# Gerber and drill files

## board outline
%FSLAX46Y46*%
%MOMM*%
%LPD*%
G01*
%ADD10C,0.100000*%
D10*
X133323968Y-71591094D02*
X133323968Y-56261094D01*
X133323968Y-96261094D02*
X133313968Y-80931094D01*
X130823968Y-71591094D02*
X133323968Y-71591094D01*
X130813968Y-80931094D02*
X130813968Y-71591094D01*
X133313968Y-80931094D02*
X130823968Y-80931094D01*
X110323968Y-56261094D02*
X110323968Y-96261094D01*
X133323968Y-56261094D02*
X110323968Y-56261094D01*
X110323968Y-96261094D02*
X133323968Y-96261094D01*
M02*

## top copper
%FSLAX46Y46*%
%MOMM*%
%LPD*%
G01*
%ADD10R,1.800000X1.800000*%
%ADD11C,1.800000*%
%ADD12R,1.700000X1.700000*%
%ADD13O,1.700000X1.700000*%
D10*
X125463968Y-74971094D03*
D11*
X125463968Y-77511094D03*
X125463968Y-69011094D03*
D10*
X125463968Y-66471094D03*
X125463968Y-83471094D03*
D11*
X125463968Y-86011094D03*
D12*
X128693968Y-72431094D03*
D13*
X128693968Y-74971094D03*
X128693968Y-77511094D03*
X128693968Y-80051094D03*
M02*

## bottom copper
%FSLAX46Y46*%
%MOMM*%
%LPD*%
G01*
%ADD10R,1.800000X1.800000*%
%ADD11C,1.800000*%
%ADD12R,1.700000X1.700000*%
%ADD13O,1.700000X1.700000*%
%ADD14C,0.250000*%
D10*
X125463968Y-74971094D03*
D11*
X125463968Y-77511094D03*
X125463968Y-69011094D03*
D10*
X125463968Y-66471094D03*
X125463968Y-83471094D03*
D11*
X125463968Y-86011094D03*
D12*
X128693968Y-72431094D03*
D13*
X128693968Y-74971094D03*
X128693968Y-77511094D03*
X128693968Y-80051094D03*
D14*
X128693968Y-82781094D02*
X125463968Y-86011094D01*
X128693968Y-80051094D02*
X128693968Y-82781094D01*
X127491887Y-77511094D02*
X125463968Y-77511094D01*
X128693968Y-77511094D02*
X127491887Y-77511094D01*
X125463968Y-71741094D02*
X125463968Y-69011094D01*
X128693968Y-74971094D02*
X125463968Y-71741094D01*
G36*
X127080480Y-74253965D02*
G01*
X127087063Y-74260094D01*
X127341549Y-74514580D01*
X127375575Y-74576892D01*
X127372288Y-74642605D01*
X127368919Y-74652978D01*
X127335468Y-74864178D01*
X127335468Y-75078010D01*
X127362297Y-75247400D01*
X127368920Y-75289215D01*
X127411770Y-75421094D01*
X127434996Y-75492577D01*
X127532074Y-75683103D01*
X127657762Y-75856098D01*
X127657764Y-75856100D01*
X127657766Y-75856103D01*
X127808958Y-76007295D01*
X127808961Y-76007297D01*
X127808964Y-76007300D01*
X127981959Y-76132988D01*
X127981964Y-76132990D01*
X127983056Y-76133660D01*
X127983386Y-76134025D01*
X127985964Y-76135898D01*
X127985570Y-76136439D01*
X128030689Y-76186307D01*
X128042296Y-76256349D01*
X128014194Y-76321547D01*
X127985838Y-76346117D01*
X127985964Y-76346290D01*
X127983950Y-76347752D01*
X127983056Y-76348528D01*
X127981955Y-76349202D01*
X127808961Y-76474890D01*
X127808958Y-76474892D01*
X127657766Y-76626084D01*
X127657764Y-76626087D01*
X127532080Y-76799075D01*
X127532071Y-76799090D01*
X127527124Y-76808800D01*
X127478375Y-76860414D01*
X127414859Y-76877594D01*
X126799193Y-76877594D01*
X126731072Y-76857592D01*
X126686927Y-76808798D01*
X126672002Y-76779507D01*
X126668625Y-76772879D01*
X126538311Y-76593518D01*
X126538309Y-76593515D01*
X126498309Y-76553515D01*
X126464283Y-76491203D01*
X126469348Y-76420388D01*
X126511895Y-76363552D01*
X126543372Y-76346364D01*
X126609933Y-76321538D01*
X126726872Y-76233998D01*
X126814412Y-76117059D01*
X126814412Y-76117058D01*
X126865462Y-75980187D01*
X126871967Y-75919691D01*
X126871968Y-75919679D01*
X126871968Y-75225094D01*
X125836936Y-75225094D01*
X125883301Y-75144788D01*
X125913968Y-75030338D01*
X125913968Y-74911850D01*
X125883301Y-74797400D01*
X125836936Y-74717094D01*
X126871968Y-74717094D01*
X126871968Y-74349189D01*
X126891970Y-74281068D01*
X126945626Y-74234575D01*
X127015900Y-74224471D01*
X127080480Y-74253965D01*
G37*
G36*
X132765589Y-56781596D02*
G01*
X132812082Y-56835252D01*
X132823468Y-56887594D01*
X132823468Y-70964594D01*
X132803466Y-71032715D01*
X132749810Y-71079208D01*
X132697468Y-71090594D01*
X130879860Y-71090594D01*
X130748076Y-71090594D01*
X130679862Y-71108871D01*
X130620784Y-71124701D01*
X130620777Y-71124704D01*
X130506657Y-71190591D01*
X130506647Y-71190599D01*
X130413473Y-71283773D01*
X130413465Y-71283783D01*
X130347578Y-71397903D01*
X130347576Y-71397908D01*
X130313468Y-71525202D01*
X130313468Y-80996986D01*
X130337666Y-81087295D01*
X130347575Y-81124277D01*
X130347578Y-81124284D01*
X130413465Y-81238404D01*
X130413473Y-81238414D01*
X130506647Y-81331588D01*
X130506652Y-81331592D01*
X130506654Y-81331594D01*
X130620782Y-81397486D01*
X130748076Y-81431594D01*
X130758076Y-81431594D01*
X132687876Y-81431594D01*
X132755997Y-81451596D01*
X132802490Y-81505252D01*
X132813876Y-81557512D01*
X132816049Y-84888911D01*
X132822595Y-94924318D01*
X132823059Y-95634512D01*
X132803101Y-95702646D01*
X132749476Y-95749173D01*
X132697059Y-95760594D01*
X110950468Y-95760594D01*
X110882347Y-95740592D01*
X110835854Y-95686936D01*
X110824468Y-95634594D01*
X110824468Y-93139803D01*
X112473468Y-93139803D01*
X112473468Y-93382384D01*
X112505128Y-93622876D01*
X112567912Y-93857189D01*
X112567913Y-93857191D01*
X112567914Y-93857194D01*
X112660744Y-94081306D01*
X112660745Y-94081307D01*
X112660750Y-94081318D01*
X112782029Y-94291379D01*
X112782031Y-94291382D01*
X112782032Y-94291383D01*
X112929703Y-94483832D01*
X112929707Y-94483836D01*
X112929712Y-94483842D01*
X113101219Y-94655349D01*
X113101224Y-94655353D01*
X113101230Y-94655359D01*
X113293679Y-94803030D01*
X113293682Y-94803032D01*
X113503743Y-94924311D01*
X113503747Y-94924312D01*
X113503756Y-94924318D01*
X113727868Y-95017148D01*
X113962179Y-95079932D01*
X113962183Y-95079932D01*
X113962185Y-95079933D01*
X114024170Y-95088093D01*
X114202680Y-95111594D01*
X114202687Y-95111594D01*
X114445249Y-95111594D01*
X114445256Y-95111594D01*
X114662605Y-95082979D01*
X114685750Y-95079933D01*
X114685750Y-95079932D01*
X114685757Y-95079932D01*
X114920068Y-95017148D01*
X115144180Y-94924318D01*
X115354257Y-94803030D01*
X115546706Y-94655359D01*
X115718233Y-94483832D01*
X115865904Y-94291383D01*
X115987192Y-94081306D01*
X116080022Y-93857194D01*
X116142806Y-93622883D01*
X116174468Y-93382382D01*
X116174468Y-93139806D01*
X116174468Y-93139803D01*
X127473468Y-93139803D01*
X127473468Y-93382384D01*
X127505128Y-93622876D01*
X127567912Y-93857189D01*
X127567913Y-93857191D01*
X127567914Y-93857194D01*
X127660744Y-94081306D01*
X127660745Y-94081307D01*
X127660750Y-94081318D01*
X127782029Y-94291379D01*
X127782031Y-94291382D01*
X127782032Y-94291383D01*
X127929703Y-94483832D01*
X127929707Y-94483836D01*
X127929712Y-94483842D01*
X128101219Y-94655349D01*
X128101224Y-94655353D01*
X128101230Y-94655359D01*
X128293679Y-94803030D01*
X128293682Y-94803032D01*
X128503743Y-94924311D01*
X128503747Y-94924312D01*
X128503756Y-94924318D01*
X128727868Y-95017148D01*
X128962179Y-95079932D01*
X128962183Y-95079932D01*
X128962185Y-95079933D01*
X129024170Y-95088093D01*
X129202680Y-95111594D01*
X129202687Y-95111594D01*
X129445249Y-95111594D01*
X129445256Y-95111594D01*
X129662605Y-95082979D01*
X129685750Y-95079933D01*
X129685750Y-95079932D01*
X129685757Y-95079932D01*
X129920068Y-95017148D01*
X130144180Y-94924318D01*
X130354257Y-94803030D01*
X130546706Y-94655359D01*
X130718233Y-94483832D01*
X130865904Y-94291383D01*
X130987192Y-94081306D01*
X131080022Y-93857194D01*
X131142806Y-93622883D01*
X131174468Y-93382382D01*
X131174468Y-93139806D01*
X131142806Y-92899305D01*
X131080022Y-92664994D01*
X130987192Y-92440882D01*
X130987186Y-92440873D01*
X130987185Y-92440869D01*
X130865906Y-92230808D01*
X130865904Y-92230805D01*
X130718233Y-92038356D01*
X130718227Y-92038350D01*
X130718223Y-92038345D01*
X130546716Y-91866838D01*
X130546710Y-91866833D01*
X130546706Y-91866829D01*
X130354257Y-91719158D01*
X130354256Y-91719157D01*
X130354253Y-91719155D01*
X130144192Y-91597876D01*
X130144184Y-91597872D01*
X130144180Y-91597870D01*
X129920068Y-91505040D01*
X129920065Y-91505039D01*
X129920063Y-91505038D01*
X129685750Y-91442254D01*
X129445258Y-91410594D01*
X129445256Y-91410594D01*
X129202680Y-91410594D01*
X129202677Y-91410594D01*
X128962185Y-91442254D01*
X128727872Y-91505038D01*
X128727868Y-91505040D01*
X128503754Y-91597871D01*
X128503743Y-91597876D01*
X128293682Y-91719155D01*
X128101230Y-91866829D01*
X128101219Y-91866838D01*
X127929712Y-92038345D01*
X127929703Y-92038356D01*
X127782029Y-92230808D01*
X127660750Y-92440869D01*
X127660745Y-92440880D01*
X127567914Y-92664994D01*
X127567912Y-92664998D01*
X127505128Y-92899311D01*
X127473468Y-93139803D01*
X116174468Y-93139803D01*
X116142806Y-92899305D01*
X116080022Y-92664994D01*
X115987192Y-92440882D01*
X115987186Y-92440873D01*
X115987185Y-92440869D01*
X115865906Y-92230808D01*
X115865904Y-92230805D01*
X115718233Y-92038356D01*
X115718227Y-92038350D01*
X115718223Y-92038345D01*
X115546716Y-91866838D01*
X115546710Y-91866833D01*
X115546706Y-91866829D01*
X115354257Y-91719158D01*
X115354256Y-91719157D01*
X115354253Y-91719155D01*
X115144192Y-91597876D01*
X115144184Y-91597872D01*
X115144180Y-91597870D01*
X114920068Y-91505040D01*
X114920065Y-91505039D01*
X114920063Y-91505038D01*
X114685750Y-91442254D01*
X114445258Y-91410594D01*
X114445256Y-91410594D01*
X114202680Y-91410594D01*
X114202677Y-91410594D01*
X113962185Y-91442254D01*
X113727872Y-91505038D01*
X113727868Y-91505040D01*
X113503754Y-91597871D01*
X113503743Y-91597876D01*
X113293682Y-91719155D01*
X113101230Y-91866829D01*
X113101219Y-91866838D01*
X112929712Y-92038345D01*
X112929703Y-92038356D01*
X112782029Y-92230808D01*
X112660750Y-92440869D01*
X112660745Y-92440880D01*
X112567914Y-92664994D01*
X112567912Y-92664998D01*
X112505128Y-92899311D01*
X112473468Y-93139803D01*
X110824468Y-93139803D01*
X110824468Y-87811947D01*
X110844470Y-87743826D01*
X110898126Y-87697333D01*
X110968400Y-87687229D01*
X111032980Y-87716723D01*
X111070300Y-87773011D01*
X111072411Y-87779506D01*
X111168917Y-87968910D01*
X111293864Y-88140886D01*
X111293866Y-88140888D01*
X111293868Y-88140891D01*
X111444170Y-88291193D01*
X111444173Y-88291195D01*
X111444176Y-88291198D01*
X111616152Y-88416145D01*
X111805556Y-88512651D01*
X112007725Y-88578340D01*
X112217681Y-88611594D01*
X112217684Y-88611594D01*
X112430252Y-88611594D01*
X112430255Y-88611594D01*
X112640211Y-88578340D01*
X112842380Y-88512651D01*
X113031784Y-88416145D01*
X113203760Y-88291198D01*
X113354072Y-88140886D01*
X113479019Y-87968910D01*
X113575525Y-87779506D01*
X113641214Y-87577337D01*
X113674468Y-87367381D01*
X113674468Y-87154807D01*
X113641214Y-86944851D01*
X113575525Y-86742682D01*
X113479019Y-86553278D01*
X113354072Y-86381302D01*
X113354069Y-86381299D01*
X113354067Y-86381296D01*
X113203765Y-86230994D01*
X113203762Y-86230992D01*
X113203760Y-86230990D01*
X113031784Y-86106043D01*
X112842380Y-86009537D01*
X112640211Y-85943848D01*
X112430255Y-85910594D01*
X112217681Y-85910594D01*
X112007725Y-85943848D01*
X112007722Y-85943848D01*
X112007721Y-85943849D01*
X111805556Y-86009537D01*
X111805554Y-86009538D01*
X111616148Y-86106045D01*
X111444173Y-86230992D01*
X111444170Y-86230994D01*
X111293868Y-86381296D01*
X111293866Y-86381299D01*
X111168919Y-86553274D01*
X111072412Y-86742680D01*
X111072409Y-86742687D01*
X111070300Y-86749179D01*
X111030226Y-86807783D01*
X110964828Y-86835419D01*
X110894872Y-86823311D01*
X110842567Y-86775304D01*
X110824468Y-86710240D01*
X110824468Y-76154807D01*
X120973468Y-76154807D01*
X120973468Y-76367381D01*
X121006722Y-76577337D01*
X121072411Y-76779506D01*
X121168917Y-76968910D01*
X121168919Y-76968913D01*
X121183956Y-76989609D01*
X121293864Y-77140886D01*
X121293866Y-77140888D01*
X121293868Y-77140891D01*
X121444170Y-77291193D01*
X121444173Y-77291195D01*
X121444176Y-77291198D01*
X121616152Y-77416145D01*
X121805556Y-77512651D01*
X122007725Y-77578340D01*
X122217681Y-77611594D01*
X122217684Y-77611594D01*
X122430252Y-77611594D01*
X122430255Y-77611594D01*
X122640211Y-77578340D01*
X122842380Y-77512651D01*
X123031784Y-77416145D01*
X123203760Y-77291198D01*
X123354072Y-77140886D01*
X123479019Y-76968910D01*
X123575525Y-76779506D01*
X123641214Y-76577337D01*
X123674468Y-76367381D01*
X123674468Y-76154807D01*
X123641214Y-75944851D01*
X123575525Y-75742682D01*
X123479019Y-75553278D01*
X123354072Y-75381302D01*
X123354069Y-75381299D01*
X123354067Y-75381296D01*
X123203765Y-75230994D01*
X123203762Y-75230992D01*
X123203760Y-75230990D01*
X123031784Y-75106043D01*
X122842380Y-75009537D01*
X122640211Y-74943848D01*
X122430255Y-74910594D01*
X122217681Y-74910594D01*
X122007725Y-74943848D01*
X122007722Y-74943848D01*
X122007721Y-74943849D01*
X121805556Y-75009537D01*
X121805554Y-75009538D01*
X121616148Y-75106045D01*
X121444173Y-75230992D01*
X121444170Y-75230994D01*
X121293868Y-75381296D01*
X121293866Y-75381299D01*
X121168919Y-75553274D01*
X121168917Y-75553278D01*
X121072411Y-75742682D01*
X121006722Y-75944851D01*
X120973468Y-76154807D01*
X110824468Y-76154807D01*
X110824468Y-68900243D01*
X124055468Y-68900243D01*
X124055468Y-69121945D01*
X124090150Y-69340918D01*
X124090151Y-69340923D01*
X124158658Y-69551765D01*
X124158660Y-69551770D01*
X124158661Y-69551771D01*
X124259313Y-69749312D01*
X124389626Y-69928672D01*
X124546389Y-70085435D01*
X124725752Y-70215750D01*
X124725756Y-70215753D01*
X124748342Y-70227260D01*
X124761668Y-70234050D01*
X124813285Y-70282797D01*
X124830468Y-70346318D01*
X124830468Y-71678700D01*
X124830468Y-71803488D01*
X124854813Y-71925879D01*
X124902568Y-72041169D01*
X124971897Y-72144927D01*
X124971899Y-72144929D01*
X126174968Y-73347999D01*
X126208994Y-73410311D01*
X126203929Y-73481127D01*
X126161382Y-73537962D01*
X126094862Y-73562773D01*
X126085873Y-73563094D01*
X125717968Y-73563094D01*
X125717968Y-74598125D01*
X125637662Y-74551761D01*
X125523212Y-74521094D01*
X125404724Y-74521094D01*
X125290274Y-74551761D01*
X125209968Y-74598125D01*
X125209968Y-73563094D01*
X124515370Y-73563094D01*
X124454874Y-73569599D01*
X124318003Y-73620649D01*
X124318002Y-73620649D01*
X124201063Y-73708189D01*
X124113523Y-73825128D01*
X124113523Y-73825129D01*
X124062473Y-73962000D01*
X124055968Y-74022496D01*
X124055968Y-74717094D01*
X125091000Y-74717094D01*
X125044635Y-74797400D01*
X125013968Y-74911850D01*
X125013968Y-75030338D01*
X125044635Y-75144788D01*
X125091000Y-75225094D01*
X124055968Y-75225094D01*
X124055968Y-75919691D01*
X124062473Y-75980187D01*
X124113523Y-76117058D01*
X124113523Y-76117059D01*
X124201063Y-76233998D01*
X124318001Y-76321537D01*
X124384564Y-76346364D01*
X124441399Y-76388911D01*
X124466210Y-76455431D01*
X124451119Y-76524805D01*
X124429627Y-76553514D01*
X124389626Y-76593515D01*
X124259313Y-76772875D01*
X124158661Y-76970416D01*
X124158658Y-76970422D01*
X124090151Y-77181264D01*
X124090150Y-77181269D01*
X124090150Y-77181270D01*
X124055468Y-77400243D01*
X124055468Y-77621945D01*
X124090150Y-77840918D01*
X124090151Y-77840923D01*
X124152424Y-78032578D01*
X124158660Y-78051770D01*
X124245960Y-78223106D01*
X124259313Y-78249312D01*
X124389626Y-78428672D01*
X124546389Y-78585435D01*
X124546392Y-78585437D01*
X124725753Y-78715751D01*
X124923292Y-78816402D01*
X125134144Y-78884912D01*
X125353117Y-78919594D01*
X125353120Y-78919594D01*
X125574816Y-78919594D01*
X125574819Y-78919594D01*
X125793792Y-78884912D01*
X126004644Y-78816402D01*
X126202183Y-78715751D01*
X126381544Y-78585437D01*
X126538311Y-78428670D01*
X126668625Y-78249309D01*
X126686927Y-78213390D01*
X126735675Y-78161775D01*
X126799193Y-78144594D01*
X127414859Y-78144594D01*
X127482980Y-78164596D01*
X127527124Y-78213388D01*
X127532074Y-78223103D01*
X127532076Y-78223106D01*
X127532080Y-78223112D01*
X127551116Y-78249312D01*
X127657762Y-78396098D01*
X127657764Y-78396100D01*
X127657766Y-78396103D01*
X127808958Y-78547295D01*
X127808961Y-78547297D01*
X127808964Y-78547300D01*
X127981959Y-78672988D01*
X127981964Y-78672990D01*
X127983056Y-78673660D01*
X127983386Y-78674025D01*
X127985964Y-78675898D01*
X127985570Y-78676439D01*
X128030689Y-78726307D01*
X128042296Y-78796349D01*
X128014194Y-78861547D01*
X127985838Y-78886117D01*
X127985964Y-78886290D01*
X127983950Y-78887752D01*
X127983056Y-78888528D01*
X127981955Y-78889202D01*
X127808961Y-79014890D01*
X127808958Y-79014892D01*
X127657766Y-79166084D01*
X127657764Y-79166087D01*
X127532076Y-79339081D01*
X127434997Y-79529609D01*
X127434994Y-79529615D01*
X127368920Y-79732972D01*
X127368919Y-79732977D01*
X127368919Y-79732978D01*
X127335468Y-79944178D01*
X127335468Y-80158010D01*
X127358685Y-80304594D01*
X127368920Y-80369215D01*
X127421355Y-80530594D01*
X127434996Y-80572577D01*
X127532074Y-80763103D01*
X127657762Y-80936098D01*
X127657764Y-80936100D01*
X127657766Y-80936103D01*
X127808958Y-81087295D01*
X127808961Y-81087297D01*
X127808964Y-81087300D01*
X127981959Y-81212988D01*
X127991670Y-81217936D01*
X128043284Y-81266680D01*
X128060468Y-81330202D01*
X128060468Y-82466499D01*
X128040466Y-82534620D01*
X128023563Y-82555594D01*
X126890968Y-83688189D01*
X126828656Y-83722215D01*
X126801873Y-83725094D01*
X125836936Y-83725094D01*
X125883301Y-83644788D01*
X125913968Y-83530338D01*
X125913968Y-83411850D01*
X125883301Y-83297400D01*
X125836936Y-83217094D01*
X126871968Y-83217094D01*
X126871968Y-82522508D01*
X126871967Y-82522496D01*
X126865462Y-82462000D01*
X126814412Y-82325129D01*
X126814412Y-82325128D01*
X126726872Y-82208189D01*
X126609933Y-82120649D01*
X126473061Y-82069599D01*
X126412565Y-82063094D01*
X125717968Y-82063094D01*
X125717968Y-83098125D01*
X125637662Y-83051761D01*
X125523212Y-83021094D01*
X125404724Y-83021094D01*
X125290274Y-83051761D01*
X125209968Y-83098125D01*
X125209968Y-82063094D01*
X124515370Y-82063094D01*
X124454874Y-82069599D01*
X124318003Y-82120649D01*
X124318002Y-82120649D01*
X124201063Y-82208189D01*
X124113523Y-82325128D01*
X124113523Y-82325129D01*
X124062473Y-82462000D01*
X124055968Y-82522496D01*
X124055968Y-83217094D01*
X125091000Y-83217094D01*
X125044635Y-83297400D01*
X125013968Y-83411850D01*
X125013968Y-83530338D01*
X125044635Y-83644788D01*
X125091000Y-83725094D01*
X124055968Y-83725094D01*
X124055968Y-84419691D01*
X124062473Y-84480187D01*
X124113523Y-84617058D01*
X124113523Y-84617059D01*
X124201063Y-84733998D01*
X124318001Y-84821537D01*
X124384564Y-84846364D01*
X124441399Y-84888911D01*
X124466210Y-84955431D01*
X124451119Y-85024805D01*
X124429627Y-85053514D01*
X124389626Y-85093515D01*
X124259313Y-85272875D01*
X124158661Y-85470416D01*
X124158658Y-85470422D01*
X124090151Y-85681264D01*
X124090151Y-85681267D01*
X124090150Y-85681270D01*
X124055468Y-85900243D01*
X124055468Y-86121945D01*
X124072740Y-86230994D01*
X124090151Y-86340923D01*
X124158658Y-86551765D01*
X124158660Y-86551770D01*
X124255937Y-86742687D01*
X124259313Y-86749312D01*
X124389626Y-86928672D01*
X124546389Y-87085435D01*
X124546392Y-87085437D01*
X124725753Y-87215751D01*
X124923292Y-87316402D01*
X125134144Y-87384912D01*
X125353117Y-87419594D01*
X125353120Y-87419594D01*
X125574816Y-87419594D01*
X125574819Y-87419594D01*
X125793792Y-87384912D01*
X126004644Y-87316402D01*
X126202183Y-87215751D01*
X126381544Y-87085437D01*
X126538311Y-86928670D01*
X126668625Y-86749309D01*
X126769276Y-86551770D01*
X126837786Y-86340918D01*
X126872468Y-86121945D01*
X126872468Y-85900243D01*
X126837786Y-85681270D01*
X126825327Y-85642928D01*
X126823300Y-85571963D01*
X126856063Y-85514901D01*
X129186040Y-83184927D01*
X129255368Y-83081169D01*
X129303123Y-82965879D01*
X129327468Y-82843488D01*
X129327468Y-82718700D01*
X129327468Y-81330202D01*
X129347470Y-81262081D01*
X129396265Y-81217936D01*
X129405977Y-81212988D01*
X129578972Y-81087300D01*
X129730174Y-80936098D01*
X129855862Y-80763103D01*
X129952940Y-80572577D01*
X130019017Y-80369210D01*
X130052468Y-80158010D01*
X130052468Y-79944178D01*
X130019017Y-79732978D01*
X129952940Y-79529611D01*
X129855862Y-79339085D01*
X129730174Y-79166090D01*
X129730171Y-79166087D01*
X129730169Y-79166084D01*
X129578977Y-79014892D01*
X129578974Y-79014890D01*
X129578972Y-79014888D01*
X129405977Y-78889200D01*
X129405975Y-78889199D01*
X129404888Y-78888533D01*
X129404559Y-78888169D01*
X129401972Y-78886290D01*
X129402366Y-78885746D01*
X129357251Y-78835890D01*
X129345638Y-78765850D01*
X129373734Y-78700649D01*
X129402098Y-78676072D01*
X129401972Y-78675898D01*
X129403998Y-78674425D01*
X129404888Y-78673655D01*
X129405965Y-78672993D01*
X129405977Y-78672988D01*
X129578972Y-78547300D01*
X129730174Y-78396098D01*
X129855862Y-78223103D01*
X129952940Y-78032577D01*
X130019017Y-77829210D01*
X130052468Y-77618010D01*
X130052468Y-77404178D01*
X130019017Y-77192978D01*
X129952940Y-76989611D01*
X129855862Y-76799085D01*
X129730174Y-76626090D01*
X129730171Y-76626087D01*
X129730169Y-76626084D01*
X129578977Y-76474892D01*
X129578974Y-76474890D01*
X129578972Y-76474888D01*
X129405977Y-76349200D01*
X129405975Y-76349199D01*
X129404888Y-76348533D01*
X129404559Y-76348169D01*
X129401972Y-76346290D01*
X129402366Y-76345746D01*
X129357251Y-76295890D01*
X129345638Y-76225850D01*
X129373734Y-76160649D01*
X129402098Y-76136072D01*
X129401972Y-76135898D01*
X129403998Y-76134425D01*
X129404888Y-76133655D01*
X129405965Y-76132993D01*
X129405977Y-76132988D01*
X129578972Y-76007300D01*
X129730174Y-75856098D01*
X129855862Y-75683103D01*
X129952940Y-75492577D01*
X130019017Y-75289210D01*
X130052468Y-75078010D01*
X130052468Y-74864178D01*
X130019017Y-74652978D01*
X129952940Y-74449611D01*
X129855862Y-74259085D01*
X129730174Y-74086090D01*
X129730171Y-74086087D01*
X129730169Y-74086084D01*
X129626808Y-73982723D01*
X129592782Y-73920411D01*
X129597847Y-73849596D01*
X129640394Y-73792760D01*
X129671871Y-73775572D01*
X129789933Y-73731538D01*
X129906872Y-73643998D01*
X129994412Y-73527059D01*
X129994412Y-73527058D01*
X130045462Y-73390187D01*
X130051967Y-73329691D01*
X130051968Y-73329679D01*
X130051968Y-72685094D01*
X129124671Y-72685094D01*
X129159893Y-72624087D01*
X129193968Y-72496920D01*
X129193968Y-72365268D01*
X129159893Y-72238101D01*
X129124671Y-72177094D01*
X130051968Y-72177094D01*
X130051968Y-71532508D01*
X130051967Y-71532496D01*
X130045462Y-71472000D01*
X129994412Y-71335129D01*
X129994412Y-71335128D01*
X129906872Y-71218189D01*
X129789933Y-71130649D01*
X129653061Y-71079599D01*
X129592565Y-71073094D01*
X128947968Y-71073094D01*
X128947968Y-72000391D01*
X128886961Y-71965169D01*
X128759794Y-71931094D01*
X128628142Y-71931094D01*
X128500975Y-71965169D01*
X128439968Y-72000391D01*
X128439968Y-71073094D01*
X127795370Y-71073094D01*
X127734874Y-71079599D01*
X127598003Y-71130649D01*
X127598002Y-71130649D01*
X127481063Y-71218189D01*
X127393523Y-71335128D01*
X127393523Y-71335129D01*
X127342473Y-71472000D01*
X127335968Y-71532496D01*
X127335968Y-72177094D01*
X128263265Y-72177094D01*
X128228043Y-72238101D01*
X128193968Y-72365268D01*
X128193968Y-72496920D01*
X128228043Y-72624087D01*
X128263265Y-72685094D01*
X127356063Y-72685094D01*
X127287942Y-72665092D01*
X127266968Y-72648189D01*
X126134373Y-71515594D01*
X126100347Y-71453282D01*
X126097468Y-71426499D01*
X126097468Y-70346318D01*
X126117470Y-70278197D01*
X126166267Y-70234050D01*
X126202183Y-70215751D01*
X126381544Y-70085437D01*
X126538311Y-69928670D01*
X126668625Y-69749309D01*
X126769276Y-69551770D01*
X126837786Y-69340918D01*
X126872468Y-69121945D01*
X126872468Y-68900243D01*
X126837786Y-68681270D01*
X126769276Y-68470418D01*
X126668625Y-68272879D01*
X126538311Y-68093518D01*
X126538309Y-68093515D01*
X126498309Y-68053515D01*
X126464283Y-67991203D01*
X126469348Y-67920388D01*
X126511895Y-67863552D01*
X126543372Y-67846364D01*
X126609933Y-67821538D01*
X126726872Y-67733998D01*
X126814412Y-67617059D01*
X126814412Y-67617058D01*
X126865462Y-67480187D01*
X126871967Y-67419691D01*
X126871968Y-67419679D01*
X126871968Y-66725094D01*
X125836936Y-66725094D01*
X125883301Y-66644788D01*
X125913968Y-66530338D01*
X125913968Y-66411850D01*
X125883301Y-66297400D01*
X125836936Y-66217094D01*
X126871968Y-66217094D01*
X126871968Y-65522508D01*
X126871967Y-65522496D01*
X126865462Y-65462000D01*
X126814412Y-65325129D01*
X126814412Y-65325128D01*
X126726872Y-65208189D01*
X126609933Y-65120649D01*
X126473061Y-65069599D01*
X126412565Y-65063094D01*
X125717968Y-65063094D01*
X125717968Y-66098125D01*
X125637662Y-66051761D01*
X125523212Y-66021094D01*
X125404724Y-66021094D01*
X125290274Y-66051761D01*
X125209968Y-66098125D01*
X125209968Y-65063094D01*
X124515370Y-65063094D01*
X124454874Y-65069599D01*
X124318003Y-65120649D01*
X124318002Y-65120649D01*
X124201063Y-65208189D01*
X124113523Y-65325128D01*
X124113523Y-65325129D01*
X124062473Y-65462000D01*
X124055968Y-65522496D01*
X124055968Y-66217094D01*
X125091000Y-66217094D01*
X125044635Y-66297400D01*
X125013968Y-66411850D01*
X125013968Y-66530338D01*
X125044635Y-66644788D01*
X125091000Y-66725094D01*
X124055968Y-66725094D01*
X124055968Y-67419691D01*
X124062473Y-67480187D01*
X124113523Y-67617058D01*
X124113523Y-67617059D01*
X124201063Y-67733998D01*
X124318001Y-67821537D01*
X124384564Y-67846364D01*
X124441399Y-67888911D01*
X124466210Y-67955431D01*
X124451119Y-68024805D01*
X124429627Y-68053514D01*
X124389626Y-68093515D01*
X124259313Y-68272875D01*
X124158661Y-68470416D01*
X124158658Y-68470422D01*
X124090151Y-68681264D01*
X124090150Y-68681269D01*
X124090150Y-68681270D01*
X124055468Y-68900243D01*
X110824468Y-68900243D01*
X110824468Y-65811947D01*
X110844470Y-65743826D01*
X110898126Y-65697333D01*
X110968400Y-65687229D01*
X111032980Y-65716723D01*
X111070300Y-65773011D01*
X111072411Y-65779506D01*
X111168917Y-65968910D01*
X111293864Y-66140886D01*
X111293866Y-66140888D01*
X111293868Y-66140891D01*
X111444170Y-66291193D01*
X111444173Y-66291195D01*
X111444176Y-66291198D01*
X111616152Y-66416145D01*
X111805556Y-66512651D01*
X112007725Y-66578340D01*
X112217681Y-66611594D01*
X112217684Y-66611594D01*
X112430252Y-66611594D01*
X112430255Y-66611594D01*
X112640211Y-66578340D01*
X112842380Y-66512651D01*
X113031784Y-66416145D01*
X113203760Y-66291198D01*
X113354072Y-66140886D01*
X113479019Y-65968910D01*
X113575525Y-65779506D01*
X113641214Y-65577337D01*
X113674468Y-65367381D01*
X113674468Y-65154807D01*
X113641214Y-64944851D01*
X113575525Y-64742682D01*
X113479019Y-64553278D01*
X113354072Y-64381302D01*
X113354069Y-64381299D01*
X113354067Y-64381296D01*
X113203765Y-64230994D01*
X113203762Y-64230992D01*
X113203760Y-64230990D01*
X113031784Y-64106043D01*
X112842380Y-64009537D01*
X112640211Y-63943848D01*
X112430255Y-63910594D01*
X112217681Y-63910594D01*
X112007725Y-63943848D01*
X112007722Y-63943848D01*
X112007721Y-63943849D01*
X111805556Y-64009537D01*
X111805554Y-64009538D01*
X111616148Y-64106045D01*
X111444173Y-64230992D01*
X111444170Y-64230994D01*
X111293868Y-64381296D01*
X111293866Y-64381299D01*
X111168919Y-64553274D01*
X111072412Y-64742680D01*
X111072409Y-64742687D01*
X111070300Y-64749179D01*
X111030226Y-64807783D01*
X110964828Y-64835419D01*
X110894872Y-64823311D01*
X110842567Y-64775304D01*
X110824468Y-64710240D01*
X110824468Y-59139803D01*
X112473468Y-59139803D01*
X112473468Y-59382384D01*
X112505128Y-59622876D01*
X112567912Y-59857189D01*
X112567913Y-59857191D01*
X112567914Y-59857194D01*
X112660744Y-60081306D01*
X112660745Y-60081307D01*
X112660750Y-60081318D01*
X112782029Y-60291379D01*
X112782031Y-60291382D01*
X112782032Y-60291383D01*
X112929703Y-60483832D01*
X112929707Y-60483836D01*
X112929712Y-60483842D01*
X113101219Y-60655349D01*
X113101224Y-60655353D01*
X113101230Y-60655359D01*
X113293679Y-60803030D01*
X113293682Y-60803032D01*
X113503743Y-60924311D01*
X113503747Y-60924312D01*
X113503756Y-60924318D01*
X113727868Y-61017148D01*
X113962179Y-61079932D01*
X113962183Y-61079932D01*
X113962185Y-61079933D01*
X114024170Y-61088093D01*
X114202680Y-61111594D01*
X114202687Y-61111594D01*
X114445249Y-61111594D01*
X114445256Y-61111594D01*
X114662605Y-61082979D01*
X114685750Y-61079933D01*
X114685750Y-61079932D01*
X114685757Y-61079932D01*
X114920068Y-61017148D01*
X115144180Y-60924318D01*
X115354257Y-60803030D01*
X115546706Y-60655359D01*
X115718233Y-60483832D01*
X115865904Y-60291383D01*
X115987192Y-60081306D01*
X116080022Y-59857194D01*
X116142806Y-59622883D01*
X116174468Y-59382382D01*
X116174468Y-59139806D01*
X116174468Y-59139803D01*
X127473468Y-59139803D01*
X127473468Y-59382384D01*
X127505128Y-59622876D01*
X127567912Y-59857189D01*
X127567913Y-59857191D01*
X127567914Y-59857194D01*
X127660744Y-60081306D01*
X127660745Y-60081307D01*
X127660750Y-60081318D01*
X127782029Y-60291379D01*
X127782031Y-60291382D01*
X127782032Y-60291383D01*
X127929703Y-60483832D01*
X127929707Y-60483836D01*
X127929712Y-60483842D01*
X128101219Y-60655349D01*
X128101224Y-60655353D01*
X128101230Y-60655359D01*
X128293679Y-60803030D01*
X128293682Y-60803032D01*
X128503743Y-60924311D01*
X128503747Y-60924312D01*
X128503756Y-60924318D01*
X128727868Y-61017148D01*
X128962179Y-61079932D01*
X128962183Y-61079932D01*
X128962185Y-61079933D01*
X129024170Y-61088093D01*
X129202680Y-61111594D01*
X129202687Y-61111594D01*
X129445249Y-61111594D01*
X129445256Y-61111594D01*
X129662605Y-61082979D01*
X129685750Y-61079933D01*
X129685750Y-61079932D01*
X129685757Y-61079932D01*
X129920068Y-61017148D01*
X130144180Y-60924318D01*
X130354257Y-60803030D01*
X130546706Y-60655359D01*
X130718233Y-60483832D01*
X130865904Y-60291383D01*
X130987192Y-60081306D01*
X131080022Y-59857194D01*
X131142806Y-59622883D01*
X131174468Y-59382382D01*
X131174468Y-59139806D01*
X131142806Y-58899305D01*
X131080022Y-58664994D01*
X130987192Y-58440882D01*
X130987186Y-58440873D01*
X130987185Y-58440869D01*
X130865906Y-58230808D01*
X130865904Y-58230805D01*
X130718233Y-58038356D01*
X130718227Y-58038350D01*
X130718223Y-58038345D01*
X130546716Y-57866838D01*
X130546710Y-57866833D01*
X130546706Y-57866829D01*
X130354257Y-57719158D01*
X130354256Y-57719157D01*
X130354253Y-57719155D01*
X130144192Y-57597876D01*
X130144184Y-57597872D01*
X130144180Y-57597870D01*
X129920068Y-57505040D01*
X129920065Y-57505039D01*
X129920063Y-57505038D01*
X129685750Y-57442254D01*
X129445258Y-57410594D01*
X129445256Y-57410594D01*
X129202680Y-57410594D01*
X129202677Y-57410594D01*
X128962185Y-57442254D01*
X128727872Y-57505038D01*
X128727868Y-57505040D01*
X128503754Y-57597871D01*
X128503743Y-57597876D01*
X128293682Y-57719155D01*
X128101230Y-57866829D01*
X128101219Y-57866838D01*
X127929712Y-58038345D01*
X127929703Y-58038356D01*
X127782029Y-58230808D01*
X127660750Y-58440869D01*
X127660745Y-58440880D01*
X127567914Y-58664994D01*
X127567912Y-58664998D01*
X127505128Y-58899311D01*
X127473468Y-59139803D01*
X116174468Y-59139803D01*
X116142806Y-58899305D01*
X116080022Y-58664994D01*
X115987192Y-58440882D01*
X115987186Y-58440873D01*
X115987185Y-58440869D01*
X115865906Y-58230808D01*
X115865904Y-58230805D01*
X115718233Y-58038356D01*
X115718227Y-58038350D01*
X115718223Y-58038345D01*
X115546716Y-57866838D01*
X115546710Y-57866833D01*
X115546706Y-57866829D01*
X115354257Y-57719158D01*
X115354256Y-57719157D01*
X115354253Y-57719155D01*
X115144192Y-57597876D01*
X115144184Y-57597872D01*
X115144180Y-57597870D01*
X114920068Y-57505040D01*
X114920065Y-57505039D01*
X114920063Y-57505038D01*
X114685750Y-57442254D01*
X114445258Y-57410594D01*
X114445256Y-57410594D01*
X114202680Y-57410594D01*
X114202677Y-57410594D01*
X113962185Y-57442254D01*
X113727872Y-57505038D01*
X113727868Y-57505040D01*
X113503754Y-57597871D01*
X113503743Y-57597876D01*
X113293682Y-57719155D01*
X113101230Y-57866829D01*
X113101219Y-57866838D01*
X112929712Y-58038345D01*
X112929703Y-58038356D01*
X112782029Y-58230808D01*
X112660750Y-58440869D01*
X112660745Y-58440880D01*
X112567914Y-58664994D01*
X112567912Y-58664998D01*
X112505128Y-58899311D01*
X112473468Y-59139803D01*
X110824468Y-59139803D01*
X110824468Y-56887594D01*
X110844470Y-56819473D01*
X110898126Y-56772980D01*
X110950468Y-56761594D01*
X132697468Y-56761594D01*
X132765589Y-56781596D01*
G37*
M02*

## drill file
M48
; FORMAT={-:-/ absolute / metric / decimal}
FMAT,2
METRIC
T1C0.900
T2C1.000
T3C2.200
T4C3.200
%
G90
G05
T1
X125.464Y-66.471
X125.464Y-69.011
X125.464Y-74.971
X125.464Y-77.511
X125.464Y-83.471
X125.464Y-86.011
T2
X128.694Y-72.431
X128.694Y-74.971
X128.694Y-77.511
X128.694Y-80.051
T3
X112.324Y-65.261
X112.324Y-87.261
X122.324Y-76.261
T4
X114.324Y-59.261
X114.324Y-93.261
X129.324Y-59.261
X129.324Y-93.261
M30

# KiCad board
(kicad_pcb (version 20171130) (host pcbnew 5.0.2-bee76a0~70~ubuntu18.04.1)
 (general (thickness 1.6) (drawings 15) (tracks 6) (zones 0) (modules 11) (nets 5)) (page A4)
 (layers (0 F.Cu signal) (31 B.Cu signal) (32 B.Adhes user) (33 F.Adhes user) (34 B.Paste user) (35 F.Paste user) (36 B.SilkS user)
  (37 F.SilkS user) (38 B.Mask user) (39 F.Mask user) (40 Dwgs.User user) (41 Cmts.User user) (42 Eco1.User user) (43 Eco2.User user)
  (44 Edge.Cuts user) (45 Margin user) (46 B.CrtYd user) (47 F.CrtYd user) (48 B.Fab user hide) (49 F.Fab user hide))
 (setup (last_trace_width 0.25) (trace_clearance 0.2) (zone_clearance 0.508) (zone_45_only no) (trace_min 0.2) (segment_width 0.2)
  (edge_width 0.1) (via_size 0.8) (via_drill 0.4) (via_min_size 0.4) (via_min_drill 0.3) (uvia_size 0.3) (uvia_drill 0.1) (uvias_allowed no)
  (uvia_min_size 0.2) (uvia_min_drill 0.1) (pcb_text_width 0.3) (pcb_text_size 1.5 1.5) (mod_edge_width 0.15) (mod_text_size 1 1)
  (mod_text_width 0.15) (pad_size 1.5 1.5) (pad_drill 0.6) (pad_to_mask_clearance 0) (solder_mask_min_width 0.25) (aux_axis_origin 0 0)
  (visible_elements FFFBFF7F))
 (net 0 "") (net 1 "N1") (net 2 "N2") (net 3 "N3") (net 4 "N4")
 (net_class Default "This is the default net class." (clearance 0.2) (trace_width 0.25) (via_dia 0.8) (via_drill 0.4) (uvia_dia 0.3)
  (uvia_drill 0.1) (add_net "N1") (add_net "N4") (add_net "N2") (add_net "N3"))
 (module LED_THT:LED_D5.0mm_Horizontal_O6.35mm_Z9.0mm (layer F.Cu) (at 125.463968 74.971094 270)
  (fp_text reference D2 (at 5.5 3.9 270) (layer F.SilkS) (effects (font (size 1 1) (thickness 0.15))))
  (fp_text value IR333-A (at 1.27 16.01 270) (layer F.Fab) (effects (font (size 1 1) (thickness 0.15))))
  (pad 1 thru_hole rect (at 0 0 270) (size 1.8 1.8) (drill 0.9) (layers *.Cu *.Mask) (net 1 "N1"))
  (pad 2 thru_hole circle (at 2.54 0 270) (size 1.8 1.8) (drill 0.9) (layers *.Cu *.Mask) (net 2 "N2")))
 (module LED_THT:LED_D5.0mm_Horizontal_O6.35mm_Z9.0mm (layer F.Cu) (at 125.463968 66.471094 270)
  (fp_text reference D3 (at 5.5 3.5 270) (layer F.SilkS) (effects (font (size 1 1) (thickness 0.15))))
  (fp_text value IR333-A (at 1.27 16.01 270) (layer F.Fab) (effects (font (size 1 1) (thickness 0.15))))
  (pad 2 thru_hole circle (at 2.54 0 270) (size 1.8 1.8) (drill 0.9) (layers *.Cu *.Mask) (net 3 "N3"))
  (pad 1 thru_hole rect (at 0 0 270) (size 1.8 1.8) (drill 0.9) (layers *.Cu *.Mask) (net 1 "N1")))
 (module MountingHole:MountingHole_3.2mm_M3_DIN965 (layer F.Cu) (at 129.323968 59.261094 180)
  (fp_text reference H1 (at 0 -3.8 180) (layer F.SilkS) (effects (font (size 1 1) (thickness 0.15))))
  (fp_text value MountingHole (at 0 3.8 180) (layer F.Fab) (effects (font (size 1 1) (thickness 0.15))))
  (pad 1 np_thru_hole circle (at 0 0 180) (size 3.2 3.2) (drill 3.2) (layers *.Cu *.Mask)))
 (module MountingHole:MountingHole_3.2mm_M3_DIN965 (layer F.Cu) (at 129.323968 93.261094 180)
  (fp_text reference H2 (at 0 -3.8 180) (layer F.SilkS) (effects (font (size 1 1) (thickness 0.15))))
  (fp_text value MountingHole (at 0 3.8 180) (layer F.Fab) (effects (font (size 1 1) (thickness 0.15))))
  (pad 1 np_thru_hole circle (at 0 0 180) (size 3.2 3.2) (drill 3.2) (layers *.Cu *.Mask)))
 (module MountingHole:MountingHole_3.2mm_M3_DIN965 (layer F.Cu) (at 114.323968 59.261094 180)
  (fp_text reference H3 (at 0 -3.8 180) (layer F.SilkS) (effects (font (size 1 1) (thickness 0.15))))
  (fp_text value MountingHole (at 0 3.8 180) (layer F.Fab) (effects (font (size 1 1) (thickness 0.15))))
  (pad 1 np_thru_hole circle (at 0 0 180) (size 3.2 3.2) (drill 3.2) (layers *.Cu *.Mask)))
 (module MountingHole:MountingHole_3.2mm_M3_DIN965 (layer F.Cu) (at 114.323968 93.261094 180)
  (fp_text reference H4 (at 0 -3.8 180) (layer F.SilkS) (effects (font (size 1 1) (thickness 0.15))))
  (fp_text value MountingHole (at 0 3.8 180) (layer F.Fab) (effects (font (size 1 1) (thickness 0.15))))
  (pad 1 np_thru_hole circle (at 0 0 180) (size 3.2 3.2) (drill 3.2) (layers *.Cu *.Mask)))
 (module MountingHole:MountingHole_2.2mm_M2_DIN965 (layer F.Cu) (at 112.323968 87.261094 180)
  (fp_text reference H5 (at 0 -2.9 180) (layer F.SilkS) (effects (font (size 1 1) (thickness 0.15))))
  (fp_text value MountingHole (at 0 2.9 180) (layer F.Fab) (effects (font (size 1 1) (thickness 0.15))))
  (pad 1 np_thru_hole circle (at 0 0 180) (size 2.2 2.2) (drill 2.2) (layers *.Cu *.Mask)))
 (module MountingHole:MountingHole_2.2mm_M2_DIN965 (layer F.Cu) (at 122.323968 76.261094 180)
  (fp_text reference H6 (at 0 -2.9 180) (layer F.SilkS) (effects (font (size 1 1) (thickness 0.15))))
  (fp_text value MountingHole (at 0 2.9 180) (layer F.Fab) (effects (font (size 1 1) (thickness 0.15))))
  (pad 1 np_thru_hole circle (at 0 0 180) (size 2.2 2.2) (drill 2.2) (layers *.Cu *.Mask)))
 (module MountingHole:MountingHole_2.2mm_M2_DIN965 (layer F.Cu) (at 112.323968 65.261094 180)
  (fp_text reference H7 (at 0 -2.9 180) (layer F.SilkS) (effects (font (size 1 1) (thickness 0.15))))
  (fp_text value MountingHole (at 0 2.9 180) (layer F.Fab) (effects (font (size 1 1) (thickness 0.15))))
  (pad 1 np_thru_hole circle (at 0 0 180) (size 2.2 2.2) (drill 2.2) (layers *.Cu *.Mask)))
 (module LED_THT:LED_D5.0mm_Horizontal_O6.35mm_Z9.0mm (layer F.Cu) (at 125.463968 83.471094 270)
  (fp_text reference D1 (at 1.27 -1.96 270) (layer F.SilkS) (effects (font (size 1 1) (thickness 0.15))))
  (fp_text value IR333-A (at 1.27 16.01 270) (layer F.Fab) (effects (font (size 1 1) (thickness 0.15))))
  (pad 1 thru_hole rect (at 0 0 270) (size 1.8 1.8) (drill 0.9) (layers *.Cu *.Mask) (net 1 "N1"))
  (pad 2 thru_hole circle (at 2.54 0 270) (size 1.8 1.8) (drill 0.9) (layers *.Cu *.Mask) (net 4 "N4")))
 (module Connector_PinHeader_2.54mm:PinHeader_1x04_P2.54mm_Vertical (layer F.Cu) (at 128.693968 72.431094)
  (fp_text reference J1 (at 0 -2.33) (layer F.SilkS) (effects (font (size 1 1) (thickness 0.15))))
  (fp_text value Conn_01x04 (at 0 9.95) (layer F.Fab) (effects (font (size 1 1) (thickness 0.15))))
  (pad 1 thru_hole rect (at 0 0) (size 1.7 1.7) (drill 1) (layers *.Cu *.Mask) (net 1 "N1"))
  (pad 2 thru_hole oval (at 0 2.54) (size 1.7 1.7) (drill 1) (layers *.Cu *.Mask) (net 3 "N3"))
  (pad 3 thru_hole oval (at 0 5.08) (size 1.7 1.7) (drill 1) (layers *.Cu *.Mask) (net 2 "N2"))
  (pad 4 thru_hole oval (at 0 7.62) (size 1.7 1.7) (drill 1) (layers *.Cu *.Mask) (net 4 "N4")))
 (gr_line (start 133.323968 71.591094) (end 133.323968 56.261094) (layer Edge.Cuts) (width 0.1))
 (gr_line (start 133.323968 96.261094) (end 133.313968 80.931094) (layer Edge.Cuts) (width 0.1))
 (gr_line (start 130.823968 71.591094) (end 133.323968 71.591094) (layer Edge.Cuts) (width 0.1))
 (gr_line (start 130.813968 80.931094) (end 130.813968 71.591094) (layer Edge.Cuts) (width 0.1))
 (gr_line (start 133.313968 80.931094) (end 130.823968 80.931094) (layer Edge.Cuts) (width 0.1))
 (gr_line (start 110.323968 56.261094) (end 110.323968 96.261094) (layer Edge.Cuts) (width 0.1))
 (gr_line (start 133.323968 56.261094) (end 110.323968 56.261094) (layer Edge.Cuts) (width 0.1))
 (gr_line (start 110.323968 96.261094) (end 133.323968 96.261094) (layer Edge.Cuts) (width 0.1))
 (segment (start 128.693968 82.781094) (end 125.463968 86.011094) (width 0.25) (layer B.Cu) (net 4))
 (segment (start 128.693968 80.051094) (end 128.693968 82.781094) (width 0.25) (layer B.Cu) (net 4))
 (segment (start 127.491887 77.511094) (end 125.463968 77.511094) (width 0.25) (layer B.Cu) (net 2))
 (segment (start 128.693968 77.511094) (end 127.491887 77.511094) (width 0.25) (layer B.Cu) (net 2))
 (segment (start 125.463968 71.741094) (end 125.463968 69.011094) (width 0.25) (layer B.Cu) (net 3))
 (segment (start 128.693968 74.971094) (end 125.463968 71.741094) (width 0.25) (layer B.Cu) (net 3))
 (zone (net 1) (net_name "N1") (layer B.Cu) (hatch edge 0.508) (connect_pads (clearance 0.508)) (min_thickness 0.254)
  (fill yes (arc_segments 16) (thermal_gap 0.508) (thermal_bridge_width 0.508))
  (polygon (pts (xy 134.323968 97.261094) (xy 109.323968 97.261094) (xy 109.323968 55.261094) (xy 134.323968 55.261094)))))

